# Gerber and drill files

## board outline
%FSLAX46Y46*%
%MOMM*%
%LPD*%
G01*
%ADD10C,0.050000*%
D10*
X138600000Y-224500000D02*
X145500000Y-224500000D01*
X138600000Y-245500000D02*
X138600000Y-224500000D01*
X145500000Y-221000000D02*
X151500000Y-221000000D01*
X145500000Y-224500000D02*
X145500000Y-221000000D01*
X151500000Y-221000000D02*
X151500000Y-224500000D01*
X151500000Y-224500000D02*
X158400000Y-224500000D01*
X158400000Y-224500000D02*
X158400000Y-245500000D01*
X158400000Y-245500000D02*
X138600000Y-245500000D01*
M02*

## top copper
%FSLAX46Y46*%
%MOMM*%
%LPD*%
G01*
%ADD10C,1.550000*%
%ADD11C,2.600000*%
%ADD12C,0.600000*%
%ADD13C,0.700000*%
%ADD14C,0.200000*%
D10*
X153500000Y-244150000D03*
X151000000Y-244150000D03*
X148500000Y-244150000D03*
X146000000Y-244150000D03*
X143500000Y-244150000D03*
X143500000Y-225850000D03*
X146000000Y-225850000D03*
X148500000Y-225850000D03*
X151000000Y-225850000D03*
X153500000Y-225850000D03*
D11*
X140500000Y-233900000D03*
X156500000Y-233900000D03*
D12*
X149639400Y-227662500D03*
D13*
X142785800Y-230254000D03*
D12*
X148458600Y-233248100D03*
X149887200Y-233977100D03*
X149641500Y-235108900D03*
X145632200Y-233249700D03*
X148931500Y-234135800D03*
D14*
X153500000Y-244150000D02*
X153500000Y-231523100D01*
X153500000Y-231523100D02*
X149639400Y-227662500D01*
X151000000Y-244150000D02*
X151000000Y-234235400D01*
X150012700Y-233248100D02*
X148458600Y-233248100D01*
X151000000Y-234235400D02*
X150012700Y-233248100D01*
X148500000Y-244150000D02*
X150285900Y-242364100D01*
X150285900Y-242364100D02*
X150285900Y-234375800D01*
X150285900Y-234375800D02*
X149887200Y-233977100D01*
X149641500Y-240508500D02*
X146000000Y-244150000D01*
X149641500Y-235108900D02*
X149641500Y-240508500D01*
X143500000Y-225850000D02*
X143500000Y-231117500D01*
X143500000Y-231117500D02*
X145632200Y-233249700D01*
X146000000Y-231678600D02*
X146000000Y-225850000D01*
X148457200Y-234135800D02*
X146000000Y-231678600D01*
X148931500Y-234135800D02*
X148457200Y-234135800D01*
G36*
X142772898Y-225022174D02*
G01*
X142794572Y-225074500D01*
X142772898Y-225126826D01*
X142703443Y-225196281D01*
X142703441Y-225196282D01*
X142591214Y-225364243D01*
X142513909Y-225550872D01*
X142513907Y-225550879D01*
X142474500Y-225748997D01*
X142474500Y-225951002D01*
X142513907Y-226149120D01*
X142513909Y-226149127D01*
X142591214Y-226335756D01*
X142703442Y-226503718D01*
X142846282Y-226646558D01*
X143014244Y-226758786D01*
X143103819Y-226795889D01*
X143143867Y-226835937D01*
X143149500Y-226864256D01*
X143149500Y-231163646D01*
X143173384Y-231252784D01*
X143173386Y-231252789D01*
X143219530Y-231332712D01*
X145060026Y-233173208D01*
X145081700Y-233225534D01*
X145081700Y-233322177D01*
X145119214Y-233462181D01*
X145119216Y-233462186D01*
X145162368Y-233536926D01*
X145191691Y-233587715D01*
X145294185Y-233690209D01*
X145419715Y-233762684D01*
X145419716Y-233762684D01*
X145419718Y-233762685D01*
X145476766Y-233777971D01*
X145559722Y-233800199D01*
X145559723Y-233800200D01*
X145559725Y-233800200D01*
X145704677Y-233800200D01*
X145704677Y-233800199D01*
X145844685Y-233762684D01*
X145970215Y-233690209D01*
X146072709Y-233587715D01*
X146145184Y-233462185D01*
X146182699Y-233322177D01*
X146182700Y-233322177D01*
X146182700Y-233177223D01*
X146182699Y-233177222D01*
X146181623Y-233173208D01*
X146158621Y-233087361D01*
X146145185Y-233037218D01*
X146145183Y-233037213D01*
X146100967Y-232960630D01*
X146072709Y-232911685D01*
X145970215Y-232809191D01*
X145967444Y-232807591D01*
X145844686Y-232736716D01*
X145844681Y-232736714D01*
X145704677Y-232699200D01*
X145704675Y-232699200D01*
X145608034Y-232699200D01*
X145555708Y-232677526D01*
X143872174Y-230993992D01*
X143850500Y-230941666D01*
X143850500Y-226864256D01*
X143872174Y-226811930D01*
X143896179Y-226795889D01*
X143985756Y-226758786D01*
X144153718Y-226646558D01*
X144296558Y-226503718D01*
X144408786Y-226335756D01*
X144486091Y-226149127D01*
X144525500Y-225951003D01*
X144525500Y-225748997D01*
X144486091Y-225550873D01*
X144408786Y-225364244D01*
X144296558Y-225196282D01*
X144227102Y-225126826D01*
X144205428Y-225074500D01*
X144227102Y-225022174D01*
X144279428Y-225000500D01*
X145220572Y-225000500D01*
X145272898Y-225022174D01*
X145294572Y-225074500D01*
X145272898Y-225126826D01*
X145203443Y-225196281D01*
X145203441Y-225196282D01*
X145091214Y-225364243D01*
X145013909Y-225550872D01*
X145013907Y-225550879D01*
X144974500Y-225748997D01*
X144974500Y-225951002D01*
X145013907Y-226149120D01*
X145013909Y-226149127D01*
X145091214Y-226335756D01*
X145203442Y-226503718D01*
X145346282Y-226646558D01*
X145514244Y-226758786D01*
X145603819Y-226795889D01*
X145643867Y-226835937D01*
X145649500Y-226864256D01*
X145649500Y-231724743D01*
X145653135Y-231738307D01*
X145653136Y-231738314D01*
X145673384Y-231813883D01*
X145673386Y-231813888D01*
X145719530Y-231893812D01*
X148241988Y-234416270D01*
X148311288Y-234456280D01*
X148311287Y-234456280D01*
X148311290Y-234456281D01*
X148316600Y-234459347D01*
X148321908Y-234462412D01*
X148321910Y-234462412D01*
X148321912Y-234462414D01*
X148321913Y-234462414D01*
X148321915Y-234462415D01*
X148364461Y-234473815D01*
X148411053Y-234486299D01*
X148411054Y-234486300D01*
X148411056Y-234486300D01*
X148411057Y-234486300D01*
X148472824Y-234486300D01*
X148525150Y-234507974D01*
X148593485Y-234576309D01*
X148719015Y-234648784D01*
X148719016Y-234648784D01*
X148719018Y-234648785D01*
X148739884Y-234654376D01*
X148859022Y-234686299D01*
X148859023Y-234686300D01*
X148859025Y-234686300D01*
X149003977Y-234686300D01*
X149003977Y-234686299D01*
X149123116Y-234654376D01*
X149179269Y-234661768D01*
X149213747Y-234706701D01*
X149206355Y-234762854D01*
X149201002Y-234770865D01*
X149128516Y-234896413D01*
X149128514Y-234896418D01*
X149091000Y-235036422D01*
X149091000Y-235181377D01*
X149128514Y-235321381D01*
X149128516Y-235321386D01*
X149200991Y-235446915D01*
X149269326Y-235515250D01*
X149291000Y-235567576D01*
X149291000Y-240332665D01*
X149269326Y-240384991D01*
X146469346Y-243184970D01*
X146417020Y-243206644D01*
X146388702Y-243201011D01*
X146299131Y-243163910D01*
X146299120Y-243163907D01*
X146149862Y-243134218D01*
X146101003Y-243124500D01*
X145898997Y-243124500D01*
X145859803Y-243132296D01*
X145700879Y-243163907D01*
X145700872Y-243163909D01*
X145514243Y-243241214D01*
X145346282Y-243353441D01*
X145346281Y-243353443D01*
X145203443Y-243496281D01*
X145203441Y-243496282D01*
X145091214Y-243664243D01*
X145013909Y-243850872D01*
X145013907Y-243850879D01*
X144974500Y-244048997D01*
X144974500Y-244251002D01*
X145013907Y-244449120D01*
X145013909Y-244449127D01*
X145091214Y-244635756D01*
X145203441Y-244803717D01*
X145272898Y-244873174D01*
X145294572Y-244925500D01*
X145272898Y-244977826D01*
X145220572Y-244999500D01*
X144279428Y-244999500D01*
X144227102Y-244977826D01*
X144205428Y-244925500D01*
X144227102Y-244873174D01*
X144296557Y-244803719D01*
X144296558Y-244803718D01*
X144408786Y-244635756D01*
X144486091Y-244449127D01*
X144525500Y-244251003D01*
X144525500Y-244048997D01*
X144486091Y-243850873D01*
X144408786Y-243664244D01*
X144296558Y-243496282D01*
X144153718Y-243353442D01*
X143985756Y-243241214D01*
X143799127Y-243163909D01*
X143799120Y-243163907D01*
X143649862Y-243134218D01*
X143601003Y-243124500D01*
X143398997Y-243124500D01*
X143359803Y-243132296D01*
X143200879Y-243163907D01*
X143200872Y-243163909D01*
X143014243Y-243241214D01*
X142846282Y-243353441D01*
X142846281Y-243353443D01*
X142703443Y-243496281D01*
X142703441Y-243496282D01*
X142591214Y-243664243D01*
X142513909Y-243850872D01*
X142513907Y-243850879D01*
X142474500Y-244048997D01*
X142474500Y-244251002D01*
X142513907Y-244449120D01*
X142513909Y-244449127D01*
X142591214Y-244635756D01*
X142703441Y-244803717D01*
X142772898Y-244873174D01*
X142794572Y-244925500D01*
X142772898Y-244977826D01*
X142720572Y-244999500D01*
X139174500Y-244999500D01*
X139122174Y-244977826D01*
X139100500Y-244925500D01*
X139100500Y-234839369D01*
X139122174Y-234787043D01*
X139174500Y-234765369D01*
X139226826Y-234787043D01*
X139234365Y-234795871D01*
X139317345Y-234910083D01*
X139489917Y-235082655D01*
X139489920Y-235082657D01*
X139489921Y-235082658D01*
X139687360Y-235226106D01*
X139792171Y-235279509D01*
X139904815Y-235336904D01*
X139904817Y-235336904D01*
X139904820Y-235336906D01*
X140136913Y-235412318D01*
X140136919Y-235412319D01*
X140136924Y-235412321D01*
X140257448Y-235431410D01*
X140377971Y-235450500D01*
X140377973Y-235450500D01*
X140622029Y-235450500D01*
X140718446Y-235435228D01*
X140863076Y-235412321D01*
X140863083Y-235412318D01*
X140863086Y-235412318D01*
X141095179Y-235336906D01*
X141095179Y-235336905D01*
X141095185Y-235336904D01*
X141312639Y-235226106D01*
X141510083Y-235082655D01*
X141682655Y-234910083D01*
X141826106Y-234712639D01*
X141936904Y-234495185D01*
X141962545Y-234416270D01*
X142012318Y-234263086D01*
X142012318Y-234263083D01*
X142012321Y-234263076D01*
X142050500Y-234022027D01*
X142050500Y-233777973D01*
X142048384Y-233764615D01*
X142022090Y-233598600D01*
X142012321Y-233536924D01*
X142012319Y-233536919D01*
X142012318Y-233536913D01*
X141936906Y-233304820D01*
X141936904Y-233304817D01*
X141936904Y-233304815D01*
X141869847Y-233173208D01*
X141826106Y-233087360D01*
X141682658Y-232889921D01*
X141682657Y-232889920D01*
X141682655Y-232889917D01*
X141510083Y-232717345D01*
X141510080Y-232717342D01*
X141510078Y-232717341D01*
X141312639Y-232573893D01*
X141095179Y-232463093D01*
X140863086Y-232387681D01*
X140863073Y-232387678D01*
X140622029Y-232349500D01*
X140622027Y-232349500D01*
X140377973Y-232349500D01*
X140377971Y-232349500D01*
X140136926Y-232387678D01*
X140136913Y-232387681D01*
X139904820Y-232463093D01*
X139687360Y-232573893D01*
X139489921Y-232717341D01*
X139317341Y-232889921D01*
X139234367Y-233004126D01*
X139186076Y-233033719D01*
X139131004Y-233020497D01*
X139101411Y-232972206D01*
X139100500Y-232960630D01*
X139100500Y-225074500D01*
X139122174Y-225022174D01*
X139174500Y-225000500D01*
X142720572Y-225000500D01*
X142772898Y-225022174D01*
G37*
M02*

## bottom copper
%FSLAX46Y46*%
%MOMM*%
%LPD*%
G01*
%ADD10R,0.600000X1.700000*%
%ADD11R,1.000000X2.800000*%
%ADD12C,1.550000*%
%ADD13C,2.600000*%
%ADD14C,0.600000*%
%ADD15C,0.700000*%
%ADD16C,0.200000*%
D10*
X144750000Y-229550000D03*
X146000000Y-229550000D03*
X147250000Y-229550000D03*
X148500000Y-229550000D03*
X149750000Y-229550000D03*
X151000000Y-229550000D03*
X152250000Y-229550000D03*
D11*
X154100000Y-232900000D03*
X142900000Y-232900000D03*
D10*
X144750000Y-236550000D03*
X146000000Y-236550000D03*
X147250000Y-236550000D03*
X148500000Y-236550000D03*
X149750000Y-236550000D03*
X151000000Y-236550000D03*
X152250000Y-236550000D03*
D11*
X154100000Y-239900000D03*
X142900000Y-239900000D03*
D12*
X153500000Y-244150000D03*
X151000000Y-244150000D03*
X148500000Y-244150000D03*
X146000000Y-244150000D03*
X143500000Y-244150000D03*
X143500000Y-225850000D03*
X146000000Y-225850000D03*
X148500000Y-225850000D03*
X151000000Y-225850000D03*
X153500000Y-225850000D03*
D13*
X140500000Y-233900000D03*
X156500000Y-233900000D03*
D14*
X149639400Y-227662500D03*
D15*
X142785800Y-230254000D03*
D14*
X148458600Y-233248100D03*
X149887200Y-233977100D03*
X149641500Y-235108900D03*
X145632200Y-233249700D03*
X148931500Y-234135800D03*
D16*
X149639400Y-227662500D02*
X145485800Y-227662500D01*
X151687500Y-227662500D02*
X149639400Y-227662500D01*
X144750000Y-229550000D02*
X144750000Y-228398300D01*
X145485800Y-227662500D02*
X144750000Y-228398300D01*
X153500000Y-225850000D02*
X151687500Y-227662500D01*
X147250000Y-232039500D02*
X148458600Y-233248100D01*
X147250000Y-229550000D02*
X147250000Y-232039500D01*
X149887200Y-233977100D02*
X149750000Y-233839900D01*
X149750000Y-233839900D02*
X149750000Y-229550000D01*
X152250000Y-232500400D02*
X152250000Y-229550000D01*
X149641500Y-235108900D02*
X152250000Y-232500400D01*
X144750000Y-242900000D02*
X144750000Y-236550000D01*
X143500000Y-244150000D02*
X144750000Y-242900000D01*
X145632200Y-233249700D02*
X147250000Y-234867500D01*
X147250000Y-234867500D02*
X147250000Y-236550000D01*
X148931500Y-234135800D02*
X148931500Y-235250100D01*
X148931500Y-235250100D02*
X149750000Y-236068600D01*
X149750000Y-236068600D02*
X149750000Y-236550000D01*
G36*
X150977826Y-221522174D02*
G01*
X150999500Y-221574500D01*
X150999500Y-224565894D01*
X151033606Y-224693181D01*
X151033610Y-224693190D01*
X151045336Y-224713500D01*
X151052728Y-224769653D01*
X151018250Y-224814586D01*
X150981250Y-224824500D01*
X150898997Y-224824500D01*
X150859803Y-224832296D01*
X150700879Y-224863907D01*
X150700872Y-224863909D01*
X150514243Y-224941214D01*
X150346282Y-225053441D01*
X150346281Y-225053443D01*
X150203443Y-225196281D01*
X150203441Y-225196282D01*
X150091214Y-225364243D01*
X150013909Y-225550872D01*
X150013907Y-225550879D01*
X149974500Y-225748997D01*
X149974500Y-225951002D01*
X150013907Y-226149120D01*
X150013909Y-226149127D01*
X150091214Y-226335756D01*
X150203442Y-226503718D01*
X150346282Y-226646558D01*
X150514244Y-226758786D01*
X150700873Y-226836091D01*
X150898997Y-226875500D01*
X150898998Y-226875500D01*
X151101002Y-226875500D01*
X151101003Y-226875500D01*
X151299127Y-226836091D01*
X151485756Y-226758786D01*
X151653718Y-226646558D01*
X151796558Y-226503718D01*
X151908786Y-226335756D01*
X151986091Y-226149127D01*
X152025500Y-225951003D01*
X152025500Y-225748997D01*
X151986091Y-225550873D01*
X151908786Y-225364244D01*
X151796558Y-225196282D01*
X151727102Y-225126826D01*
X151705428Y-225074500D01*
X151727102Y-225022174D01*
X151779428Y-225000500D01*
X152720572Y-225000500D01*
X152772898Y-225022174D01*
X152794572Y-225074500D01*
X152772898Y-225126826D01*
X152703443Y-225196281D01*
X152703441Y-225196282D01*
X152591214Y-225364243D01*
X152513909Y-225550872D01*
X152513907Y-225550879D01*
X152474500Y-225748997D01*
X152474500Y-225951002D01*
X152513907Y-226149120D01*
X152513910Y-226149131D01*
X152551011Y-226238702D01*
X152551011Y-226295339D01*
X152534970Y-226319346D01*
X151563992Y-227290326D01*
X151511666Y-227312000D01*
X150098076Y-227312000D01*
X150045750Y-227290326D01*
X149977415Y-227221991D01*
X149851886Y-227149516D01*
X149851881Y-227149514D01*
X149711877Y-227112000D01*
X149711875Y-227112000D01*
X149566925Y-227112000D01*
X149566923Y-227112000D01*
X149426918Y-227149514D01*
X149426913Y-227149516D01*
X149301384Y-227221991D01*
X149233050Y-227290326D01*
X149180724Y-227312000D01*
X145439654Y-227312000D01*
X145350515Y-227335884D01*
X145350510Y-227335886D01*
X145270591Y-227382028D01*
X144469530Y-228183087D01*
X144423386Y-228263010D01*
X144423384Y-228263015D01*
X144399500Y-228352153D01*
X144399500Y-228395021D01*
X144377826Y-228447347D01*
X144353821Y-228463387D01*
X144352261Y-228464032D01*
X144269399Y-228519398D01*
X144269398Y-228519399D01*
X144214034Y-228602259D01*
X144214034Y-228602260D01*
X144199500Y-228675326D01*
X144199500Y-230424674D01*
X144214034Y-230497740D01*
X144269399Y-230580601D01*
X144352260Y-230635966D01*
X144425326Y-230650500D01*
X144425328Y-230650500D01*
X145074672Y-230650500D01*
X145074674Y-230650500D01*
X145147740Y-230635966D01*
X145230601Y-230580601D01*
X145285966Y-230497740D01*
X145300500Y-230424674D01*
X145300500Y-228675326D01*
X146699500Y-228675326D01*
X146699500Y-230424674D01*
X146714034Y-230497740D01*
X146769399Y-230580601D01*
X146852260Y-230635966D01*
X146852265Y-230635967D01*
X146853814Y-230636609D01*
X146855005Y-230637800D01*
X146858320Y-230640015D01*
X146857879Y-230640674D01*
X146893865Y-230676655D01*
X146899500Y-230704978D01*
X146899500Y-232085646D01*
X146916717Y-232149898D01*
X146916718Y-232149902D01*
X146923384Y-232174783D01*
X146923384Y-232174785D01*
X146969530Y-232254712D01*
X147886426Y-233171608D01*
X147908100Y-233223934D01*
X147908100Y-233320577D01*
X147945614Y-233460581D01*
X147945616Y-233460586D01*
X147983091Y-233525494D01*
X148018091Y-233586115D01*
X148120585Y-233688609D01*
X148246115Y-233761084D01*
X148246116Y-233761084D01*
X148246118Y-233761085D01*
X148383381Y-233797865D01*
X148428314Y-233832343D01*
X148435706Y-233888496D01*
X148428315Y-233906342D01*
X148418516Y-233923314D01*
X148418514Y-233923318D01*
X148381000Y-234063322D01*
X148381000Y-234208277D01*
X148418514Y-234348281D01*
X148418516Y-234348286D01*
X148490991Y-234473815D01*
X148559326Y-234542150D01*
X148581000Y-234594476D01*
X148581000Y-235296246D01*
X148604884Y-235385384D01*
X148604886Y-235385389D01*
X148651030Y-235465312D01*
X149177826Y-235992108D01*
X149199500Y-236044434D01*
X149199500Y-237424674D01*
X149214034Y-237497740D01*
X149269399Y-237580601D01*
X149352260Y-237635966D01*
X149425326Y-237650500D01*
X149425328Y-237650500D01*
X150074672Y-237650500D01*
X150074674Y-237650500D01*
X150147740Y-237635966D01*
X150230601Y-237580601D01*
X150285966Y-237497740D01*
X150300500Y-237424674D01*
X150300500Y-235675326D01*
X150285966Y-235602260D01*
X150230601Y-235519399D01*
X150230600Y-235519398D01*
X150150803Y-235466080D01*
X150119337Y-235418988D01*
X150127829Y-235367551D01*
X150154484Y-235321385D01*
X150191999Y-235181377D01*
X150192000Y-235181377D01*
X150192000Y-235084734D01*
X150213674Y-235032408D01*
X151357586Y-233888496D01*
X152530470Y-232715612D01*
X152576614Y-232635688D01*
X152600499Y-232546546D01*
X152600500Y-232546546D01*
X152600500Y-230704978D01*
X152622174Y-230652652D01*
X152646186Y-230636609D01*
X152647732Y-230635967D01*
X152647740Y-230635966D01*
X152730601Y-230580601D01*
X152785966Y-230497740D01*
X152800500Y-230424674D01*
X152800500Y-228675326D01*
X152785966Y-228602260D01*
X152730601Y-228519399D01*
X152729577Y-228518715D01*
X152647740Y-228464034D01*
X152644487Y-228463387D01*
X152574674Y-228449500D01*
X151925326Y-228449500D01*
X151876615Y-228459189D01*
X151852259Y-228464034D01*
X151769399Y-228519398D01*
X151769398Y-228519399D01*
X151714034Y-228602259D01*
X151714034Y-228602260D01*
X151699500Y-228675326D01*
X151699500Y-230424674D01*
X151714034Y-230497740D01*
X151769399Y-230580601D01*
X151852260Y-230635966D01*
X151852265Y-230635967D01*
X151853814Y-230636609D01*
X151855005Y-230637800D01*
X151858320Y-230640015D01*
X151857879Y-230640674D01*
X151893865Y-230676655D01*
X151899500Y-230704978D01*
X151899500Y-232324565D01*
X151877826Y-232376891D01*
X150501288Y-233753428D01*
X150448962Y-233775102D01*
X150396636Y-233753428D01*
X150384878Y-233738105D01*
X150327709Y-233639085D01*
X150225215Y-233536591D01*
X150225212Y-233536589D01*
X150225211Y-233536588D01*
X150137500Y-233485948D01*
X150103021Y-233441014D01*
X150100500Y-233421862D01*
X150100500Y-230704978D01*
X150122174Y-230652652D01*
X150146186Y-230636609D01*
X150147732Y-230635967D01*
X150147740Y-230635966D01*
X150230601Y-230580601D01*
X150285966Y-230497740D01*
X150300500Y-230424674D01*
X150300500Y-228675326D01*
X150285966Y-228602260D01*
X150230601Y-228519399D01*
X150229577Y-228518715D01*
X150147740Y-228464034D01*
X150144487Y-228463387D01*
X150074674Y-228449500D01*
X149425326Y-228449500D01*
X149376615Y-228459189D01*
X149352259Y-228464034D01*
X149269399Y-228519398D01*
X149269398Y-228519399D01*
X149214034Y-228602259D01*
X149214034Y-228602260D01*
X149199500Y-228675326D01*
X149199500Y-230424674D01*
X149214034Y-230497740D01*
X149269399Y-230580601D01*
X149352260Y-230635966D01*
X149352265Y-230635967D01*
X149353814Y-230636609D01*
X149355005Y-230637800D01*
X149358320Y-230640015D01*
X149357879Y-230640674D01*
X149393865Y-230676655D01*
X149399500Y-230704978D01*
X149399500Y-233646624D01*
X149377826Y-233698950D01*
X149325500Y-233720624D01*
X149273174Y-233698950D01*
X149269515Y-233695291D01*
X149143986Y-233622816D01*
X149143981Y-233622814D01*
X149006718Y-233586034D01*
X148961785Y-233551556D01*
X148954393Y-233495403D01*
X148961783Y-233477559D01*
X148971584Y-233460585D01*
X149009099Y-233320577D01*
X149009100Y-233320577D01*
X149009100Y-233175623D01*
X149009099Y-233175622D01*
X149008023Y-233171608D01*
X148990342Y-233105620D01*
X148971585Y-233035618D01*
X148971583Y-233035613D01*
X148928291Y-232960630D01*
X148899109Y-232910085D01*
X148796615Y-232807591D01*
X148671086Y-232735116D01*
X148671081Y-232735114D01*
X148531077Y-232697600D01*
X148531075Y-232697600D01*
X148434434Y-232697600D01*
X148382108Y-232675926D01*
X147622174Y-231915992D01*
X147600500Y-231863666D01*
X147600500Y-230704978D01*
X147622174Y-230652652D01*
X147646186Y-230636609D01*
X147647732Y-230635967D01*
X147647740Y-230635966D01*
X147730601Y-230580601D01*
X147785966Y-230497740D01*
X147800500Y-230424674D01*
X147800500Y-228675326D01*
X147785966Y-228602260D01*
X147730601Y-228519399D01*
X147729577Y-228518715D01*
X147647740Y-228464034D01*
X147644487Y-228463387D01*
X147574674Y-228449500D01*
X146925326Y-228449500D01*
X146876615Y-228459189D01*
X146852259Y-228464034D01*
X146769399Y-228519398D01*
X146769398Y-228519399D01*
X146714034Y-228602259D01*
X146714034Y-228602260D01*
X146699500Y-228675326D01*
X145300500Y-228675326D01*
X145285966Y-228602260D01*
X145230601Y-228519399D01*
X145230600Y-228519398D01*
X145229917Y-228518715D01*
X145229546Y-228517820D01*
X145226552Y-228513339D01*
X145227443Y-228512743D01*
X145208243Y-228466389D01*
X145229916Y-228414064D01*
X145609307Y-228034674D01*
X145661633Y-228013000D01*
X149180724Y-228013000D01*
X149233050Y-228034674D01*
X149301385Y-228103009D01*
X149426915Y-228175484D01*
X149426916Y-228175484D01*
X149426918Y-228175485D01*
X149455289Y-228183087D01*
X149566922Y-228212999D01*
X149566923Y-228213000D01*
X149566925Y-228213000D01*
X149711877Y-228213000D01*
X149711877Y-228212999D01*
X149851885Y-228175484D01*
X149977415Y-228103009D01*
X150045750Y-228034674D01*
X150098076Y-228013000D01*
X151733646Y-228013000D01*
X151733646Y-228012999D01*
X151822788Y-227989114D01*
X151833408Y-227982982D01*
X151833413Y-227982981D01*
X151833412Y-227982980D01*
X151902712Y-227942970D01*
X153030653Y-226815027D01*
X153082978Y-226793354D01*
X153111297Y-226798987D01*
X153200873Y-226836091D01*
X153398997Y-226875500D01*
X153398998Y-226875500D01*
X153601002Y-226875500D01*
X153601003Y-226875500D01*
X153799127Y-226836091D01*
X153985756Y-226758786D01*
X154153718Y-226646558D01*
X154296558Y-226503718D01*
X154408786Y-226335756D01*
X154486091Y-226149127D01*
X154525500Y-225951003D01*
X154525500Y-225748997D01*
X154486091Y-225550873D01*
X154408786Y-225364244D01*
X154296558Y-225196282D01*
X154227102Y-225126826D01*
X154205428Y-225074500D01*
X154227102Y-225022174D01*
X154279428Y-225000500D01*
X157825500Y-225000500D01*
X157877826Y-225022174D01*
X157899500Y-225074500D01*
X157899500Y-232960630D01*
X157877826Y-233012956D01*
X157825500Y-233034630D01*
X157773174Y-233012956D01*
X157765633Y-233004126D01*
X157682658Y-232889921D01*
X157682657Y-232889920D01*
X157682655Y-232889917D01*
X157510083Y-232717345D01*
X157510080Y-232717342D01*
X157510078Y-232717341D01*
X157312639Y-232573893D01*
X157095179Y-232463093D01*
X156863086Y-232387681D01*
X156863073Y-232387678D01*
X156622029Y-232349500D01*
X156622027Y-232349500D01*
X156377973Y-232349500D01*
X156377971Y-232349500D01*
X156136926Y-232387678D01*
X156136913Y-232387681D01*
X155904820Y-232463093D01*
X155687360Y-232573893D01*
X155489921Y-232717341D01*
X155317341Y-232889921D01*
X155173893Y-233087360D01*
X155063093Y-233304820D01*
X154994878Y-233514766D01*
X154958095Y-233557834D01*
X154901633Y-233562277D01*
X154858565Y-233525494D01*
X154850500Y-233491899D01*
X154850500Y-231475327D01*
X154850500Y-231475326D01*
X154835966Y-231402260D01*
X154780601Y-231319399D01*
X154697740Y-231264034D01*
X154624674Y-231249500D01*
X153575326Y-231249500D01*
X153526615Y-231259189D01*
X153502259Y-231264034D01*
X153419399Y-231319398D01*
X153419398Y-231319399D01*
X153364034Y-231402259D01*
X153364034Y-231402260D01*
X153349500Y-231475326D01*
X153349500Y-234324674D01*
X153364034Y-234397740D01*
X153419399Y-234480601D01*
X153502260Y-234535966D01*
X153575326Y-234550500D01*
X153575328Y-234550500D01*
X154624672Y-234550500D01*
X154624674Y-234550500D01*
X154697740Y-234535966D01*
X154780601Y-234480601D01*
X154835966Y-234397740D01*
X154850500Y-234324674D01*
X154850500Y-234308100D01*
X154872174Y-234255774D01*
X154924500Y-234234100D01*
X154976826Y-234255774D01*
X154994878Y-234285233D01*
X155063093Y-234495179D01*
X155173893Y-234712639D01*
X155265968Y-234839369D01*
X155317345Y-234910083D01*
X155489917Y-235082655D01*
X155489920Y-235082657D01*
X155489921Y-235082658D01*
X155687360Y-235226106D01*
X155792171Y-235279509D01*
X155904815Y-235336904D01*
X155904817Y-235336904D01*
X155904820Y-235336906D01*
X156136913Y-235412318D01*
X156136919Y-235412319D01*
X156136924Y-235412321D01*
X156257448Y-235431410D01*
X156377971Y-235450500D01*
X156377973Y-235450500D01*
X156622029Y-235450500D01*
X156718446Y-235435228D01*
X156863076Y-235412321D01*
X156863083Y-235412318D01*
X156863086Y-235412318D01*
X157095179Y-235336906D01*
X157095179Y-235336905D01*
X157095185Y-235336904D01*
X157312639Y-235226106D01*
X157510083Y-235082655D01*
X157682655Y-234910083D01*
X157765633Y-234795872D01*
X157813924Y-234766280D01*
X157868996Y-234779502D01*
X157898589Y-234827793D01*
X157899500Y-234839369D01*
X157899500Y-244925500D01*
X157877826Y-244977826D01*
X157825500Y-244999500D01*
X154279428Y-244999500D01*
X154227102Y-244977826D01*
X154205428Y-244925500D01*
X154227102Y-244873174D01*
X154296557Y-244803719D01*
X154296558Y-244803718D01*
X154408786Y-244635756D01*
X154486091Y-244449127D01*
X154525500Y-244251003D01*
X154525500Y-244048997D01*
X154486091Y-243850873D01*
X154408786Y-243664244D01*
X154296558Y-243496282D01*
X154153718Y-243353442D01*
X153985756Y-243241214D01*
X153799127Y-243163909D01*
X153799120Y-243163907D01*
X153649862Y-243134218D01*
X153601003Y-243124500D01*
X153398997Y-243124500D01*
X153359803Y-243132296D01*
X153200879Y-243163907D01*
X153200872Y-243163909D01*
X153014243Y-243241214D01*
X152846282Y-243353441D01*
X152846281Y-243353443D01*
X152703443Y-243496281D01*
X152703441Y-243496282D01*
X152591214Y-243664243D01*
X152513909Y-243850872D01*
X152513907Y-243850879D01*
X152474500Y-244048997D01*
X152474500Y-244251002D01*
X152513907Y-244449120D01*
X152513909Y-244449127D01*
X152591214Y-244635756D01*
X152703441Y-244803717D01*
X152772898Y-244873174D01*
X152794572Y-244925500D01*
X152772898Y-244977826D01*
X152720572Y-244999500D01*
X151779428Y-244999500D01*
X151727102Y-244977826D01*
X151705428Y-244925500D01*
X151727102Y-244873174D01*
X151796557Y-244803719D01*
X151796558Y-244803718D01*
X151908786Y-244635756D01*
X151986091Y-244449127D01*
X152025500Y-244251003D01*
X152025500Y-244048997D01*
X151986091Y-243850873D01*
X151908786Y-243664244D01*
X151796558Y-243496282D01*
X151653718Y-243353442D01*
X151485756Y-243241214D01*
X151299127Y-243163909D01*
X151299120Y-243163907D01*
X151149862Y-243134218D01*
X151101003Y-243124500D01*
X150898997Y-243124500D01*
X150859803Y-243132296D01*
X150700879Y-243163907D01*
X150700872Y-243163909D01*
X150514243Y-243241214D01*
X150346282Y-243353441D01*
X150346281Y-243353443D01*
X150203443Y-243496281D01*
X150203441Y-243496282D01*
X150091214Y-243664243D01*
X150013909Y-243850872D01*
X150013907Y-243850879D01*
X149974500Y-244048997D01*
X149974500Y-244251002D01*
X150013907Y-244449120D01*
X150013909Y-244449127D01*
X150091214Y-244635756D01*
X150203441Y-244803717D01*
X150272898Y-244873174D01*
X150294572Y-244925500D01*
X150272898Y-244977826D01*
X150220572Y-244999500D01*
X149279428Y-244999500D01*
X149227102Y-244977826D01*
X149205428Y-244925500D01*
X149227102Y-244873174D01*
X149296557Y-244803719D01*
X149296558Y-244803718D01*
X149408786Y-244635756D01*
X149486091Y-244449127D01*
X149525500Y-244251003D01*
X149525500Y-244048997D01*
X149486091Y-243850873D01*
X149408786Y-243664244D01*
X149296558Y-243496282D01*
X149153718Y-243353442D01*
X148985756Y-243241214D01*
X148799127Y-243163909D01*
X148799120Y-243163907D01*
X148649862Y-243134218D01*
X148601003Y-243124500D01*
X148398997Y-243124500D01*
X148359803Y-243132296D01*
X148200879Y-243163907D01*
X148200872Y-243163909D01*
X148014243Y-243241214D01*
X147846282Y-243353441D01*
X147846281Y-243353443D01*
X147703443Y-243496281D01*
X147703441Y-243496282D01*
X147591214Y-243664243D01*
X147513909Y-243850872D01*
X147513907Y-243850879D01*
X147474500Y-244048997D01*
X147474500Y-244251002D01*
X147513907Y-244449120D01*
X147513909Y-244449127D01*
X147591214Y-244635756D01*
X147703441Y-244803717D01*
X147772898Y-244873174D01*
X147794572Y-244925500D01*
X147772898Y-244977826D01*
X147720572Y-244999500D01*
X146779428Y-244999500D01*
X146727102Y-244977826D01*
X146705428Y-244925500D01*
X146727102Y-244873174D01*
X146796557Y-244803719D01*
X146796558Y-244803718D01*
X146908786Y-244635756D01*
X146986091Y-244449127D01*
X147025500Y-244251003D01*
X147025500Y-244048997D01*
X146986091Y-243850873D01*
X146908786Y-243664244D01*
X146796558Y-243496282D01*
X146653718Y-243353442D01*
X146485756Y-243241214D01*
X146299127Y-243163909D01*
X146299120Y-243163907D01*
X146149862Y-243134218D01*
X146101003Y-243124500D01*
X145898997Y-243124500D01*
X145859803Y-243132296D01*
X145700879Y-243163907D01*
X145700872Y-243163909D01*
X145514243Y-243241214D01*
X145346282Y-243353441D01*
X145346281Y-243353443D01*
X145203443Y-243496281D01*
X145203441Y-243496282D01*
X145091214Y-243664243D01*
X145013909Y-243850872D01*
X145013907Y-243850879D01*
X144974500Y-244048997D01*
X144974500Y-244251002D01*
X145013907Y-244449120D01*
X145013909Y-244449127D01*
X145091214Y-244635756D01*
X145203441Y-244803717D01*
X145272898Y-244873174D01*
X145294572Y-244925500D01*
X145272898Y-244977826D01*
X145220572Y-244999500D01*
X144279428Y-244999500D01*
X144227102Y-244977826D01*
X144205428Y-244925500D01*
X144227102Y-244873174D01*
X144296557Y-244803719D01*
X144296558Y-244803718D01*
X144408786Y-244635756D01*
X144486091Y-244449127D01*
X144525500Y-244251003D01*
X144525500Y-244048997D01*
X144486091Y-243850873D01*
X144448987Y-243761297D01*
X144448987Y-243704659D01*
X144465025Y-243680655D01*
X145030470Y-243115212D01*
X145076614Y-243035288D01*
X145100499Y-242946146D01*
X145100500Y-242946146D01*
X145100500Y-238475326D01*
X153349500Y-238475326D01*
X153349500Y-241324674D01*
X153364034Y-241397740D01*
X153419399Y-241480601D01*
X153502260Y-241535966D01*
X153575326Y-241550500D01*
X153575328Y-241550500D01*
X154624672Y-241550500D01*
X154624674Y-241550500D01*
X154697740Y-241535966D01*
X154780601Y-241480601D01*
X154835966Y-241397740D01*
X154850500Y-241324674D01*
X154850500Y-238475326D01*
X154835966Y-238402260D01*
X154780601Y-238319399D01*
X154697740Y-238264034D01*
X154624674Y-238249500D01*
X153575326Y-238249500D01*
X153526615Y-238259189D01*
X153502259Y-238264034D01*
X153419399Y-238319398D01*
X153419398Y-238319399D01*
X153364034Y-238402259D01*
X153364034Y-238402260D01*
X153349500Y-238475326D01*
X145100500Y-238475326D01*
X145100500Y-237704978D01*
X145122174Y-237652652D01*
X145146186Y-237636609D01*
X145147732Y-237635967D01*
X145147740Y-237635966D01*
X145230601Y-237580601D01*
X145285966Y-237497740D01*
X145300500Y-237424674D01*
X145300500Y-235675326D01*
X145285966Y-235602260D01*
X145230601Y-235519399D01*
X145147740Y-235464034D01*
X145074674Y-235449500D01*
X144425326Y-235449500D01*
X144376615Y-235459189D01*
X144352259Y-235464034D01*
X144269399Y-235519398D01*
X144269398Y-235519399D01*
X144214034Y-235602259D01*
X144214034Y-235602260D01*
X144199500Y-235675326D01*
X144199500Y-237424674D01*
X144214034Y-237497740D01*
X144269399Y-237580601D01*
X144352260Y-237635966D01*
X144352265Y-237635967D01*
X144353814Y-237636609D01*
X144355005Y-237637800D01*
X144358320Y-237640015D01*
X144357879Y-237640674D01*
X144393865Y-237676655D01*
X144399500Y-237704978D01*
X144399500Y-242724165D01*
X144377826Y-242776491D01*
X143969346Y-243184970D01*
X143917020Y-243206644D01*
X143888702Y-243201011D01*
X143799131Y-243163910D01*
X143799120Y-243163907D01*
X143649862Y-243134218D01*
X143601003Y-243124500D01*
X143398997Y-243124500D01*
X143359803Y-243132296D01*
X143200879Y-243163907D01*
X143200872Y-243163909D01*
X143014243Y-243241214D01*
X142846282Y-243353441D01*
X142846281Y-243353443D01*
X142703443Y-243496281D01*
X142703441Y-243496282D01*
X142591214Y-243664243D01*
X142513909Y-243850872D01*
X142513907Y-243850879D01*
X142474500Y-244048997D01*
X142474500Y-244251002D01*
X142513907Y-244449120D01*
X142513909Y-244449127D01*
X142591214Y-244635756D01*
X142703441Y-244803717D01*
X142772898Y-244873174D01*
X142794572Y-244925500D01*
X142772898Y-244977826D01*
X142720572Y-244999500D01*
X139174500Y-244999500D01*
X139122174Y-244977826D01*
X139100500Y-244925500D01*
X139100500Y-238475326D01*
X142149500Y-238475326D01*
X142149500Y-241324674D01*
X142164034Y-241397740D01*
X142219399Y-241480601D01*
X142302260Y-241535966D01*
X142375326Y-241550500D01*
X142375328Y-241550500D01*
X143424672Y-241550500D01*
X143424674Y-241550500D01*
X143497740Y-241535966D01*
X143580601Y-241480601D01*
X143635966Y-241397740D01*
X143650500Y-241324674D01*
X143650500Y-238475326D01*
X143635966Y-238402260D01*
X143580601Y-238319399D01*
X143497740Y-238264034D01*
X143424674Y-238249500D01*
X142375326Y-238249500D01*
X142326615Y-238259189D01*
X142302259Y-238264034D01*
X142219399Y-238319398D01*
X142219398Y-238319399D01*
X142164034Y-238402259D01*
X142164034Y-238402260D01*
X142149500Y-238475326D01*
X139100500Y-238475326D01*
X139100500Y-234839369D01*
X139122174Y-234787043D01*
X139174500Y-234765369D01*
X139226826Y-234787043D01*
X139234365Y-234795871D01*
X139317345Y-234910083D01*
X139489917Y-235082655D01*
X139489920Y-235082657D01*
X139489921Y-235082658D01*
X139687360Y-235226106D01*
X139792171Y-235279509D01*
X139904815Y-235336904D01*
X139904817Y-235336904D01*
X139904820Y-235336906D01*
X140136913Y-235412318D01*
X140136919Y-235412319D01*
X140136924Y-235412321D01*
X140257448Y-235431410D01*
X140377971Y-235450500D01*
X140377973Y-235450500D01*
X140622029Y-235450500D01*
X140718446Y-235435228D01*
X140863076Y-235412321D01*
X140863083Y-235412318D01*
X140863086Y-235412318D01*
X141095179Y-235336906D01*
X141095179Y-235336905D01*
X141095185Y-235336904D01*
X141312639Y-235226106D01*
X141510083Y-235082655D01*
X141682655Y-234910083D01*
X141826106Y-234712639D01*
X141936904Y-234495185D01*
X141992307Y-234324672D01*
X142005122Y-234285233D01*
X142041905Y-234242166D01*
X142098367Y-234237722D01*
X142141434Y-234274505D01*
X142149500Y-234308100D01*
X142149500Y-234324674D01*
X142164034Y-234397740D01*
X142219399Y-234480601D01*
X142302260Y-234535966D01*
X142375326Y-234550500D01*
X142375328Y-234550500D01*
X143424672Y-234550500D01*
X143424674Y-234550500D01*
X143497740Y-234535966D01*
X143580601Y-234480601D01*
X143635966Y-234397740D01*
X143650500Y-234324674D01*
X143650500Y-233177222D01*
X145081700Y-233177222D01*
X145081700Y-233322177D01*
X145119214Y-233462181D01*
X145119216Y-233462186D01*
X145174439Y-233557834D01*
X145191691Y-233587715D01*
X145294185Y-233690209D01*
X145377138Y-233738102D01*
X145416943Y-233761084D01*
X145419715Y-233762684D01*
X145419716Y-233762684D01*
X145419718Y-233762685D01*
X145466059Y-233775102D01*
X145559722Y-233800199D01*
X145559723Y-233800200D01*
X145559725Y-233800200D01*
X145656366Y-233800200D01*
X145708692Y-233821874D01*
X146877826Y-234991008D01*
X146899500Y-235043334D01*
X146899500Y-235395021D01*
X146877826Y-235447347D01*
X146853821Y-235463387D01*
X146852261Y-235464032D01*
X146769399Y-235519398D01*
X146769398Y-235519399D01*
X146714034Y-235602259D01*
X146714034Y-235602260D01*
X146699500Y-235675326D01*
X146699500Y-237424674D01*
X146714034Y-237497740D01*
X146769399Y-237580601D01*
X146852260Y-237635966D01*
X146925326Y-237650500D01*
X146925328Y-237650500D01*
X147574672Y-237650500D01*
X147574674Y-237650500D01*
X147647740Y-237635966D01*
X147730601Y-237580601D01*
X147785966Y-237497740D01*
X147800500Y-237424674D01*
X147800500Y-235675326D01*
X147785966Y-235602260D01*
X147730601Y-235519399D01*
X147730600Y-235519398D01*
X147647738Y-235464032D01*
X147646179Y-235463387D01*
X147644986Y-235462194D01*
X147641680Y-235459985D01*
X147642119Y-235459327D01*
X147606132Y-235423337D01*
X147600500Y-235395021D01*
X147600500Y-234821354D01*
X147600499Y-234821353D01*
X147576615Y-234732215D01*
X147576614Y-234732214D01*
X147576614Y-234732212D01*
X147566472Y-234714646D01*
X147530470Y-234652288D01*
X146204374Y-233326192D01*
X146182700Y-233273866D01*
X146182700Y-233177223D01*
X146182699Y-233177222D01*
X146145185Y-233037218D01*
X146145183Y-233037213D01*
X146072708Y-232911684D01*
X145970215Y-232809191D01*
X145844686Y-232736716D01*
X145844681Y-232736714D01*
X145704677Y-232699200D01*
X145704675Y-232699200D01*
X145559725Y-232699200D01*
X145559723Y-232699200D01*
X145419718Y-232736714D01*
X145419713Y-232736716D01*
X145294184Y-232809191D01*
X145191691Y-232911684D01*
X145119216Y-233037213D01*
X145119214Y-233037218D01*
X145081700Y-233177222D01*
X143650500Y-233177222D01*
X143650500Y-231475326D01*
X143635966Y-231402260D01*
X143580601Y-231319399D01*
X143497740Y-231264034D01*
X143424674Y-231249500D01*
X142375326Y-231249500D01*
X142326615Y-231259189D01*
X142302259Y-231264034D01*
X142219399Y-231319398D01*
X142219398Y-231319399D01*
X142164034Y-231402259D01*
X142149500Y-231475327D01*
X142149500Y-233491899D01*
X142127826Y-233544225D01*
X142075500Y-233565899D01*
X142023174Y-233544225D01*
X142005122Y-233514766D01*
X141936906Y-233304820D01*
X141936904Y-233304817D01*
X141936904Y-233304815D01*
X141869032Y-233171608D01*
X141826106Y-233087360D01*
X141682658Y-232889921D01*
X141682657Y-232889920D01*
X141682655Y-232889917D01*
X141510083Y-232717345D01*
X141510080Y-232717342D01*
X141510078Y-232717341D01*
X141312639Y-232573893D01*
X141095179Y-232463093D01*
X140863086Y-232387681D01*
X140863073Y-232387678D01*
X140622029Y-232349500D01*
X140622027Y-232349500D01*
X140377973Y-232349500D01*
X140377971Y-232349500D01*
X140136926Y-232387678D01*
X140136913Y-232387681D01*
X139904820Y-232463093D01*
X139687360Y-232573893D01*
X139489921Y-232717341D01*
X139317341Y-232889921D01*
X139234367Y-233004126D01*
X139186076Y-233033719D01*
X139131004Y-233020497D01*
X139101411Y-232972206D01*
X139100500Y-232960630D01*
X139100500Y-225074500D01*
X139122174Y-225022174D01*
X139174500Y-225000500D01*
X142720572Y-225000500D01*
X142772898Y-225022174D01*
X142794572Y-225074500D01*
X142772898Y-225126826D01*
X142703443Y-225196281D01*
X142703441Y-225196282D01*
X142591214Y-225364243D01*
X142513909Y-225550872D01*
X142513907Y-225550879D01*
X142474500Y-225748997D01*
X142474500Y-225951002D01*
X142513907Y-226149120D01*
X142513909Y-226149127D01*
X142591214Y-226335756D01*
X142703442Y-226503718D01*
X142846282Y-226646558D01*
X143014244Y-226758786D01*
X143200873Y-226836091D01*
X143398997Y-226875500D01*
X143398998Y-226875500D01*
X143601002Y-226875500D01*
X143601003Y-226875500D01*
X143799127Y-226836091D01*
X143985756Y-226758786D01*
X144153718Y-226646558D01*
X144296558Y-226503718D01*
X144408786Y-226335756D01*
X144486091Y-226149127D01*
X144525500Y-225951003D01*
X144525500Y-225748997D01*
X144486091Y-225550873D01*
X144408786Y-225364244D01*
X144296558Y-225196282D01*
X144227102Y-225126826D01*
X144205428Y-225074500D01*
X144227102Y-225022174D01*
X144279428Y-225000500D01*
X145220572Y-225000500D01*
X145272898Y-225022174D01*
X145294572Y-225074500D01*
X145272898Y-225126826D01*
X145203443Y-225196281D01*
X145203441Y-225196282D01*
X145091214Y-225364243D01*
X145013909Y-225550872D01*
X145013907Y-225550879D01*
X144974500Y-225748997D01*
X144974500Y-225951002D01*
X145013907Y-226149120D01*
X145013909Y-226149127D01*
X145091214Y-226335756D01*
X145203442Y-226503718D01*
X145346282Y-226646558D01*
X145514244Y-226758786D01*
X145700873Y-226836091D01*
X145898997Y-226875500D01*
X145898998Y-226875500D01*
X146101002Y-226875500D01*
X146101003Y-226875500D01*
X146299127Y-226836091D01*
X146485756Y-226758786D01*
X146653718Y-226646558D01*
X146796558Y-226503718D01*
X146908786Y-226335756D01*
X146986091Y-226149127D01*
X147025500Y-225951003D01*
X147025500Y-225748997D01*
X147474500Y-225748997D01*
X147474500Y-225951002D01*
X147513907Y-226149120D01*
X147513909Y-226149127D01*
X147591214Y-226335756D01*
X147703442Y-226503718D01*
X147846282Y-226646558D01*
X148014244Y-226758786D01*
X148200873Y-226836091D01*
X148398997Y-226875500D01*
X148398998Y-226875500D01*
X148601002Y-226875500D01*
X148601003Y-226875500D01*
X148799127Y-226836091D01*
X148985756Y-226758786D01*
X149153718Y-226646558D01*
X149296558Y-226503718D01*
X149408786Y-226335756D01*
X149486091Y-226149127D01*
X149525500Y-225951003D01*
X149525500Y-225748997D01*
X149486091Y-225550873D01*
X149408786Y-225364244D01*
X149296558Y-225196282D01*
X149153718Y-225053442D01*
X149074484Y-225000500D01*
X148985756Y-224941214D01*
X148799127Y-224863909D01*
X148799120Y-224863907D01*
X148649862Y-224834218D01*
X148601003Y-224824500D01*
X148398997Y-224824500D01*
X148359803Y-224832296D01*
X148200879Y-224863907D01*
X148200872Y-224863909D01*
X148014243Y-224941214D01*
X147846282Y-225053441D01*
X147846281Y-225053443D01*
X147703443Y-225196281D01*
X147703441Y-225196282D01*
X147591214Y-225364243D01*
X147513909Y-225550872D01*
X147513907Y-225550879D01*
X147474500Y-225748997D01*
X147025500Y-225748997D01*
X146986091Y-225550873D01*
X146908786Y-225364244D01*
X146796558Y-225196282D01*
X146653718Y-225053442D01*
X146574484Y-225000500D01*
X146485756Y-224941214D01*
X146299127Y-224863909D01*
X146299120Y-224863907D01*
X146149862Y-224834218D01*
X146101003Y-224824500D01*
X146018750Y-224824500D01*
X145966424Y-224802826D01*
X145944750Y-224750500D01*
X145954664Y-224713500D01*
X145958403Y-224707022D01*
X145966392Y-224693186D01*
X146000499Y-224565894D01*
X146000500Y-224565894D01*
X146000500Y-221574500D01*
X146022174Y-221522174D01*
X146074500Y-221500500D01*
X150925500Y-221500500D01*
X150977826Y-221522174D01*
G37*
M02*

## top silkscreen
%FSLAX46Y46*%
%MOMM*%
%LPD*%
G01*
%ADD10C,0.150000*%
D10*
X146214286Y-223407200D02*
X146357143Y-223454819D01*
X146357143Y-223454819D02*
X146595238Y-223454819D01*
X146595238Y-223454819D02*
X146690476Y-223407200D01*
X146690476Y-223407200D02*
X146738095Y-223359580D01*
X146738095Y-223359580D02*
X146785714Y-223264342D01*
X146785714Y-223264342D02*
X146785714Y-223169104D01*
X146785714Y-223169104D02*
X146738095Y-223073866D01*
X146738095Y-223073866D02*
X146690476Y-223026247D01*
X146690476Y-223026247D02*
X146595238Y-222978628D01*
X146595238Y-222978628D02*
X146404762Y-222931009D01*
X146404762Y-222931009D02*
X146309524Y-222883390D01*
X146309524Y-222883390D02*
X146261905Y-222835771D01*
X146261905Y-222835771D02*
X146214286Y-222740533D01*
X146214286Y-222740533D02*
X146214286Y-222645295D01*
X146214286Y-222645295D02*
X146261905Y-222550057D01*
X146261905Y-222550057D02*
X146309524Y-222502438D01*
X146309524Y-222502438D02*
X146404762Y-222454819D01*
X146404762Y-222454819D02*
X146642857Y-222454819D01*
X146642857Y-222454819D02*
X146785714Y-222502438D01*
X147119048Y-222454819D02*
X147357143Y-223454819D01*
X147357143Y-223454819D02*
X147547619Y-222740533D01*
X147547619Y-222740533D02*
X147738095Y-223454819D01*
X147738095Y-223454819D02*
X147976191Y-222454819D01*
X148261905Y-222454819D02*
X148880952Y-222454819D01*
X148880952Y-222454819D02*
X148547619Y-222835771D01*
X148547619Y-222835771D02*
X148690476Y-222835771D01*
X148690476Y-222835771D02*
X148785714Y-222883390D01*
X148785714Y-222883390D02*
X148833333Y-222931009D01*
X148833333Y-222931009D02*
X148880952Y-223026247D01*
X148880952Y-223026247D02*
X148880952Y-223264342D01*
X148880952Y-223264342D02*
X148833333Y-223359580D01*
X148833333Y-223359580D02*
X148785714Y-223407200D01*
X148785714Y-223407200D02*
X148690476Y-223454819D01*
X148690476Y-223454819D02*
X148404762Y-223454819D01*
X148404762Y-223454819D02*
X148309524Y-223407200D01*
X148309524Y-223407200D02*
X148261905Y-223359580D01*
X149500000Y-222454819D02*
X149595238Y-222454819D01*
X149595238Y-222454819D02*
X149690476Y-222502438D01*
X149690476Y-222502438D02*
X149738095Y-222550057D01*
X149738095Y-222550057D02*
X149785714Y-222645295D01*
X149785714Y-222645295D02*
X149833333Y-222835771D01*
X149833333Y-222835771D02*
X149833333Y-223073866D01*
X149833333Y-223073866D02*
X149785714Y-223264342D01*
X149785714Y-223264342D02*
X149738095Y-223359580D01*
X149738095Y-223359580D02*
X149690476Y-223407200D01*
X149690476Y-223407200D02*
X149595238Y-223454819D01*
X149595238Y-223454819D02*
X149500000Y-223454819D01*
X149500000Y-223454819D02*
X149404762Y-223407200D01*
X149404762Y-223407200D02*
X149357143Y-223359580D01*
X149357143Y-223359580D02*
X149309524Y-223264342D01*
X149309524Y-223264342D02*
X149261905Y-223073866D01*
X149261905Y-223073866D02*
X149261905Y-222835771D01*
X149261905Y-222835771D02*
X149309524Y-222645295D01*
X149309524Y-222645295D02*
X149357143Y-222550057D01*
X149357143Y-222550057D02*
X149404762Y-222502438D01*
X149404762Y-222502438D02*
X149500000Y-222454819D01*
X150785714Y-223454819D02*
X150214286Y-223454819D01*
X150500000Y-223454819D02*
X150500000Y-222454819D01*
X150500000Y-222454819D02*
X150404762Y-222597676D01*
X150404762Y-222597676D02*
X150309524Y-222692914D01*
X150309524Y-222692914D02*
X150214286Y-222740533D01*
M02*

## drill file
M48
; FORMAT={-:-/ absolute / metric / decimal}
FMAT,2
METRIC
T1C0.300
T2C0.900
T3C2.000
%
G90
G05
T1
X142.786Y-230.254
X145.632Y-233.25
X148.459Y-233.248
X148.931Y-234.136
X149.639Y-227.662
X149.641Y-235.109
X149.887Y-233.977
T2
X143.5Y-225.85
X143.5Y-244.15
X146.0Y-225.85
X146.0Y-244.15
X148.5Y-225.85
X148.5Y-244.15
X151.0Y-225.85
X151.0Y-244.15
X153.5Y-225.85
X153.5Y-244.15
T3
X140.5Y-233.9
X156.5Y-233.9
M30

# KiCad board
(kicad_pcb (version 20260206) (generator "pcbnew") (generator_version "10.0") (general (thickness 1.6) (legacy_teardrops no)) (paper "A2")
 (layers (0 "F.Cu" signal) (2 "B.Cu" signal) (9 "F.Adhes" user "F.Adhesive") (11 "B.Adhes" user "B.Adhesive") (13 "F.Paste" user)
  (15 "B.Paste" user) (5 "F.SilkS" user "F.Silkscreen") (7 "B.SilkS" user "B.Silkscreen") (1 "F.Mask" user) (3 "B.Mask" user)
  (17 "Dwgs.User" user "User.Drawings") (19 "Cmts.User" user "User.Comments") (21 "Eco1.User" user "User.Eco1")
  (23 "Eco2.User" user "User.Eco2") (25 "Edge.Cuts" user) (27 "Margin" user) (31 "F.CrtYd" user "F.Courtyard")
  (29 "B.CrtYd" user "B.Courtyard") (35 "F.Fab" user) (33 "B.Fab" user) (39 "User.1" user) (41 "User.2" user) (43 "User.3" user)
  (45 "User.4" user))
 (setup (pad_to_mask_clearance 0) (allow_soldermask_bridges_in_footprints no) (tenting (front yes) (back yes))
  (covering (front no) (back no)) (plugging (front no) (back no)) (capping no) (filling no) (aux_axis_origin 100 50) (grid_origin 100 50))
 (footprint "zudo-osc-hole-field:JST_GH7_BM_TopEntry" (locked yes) (layer "B.Cu") (at 148.5 229.55 180)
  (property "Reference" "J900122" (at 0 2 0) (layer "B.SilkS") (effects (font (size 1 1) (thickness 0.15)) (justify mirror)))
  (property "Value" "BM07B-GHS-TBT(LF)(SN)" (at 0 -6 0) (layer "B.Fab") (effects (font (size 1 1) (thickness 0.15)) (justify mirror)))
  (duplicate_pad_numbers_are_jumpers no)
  (pad "1" smd rect (at 3.75 0 180) (size 0.6 1.7) (layers "B.Cu" "B.Mask" "B.Paste") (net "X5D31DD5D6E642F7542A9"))
  (pad "2" smd rect (at 2.5 0 180) (size 0.6 1.7) (layers "B.Cu" "B.Mask" "B.Paste") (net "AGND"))
  (pad "3" smd rect (at 1.25 0 180) (size 0.6 1.7) (layers "B.Cu" "B.Mask" "B.Paste") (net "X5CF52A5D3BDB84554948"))
  (pad "4" smd rect (at 0 0 180) (size 0.6 1.7) (layers "B.Cu" "B.Mask" "B.Paste") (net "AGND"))
  (pad "5" smd rect (at -1.25 0 180) (size 0.6 1.7) (layers "B.Cu" "B.Mask" "B.Paste") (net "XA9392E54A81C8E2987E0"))
  (pad "6" smd rect (at -2.5 0 180) (size 0.6 1.7) (layers "B.Cu" "B.Mask" "B.Paste") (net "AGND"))
  (pad "7" smd rect (at -3.75 0 180) (size 0.6 1.7) (layers "B.Cu" "B.Mask" "B.Paste") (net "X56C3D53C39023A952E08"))
  (pad "MP1" smd rect (at -5.6 -3.35 180) (size 1 2.8) (layers "B.Cu" "B.Mask" "B.Paste") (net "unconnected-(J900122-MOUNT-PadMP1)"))
  (pad "MP2" smd rect (at 5.6 -3.35 180) (size 1 2.8) (layers "B.Cu" "B.Mask" "B.Paste") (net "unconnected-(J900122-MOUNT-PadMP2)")))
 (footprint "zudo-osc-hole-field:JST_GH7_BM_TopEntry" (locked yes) (layer "B.Cu") (at 148.5 236.55 180)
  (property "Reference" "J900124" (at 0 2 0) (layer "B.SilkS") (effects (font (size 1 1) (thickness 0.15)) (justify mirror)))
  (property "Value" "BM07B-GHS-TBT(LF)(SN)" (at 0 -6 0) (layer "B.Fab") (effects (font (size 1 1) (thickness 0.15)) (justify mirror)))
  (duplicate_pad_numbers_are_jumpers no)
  (pad "1" smd rect (at 3.75 0 180) (size 0.6 1.7) (layers "B.Cu" "B.Mask" "B.Paste") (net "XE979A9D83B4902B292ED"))
  (pad "2" smd rect (at 2.5 0 180) (size 0.6 1.7) (layers "B.Cu" "B.Mask" "B.Paste") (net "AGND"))
  (pad "3" smd rect (at 1.25 0 180) (size 0.6 1.7) (layers "B.Cu" "B.Mask" "B.Paste") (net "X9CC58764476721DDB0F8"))
  (pad "4" smd rect (at 0 0 180) (size 0.6 1.7) (layers "B.Cu" "B.Mask" "B.Paste") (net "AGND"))
  (pad "5" smd rect (at -1.25 0 180) (size 0.6 1.7) (layers "B.Cu" "B.Mask" "B.Paste") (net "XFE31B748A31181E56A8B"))
  (pad "6" smd rect (at -2.5 0 180) (size 0.6 1.7) (layers "B.Cu" "B.Mask" "B.Paste") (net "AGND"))
  (pad "7" smd rect (at -3.75 0 180) (size 0.6 1.7) (layers "B.Cu" "B.Mask" "B.Paste") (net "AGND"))
  (pad "MP1" smd rect (at -5.6 -3.35 180) (size 1 2.8) (layers "B.Cu" "B.Mask" "B.Paste") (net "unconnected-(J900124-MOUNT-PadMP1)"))
  (pad "MP2" smd rect (at 5.6 -3.35 180) (size 1 2.8) (layers "B.Cu" "B.Mask" "B.Paste") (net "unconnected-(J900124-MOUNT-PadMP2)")))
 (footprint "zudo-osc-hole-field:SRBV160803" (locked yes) (layer "F.Cu") (at 148.5 235)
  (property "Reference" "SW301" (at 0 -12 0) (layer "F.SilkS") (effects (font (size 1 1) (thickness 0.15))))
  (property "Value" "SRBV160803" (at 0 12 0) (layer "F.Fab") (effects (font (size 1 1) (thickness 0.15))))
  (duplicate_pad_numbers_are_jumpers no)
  (pad "1" thru_hole circle (at 5 9.15) (size 1.55 1.55) (drill 0.9) (layers "*.Cu" "*.Mask") (remove_unused_layers no)
   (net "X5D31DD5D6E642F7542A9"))
  (pad "2" thru_hole circle (at 2.5 9.15) (size 1.55 1.55) (drill 0.9) (layers "*.Cu" "*.Mask") (remove_unused_layers no)
   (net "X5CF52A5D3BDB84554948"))
  (pad "3" thru_hole circle (at 0 9.15) (size 1.55 1.55) (drill 0.9) (layers "*.Cu" "*.Mask") (remove_unused_layers no)
   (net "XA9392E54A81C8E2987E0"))
  (pad "4" thru_hole circle (at -2.5 9.15) (size 1.55 1.55) (drill 0.9) (layers "*.Cu" "*.Mask") (remove_unused_layers no)
   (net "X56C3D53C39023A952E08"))
  (pad "5" thru_hole circle (at -5 9.15) (size 1.55 1.55) (drill 0.9) (layers "*.Cu" "*.Mask") (remove_unused_layers no)
   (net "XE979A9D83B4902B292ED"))
  (pad "6" thru_hole circle (at -5 -9.15) (size 1.55 1.55) (drill 0.9) (layers "*.Cu" "*.Mask") (remove_unused_layers no)
   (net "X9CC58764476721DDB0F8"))
  (pad "7" thru_hole circle (at -2.5 -9.15) (size 1.55 1.55) (drill 0.9) (layers "*.Cu" "*.Mask") (remove_unused_layers no)
   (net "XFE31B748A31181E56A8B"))
  (pad "8" thru_hole circle (at 0 -9.15) (size 1.55 1.55) (drill 0.9) (layers "*.Cu" "*.Mask") (remove_unused_layers no)
   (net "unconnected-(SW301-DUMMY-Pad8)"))
  (pad "9" thru_hole circle (at 2.5 -9.15) (size 1.55 1.55) (drill 0.9) (layers "*.Cu" "*.Mask") (remove_unused_layers no)
   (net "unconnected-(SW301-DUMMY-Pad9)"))
  (pad "10" thru_hole circle (at 5 -9.15) (size 1.55 1.55) (drill 0.9) (layers "*.Cu" "*.Mask") (remove_unused_layers no)
   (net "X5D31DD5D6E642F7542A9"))
  (pad "MP1" thru_hole circle (at -8 -1.1) (size 2.6 2.6) (drill 2) (layers "*.Cu" "*.Mask") (remove_unused_layers no)
   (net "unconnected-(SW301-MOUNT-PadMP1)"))
  (pad "MP2" thru_hole circle (at 8 -1.1) (size 2.6 2.6) (drill 2) (layers "*.Cu" "*.Mask") (remove_unused_layers no)
   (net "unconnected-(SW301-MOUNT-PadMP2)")))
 (gr_line (start 138.6 224.5) (end 145.5 224.5) (stroke (width 0.05) (type default)) (layer "Edge.Cuts"))
 (gr_line (start 138.6 245.5) (end 138.6 224.5) (stroke (width 0.05) (type default)) (layer "Edge.Cuts"))
 (gr_line (start 145.5 221) (end 151.5 221) (stroke (width 0.05) (type default)) (layer "Edge.Cuts"))
 (gr_line (start 145.5 224.5) (end 145.5 221) (stroke (width 0.05) (type default)) (layer "Edge.Cuts"))
 (gr_line (start 151.5 221) (end 151.5 224.5) (stroke (width 0.05) (type default)) (layer "Edge.Cuts"))
 (gr_line (start 151.5 224.5) (end 158.4 224.5) (stroke (width 0.05) (type default)) (layer "Edge.Cuts"))
 (gr_line (start 158.4 224.5) (end 158.4 245.5) (stroke (width 0.05) (type default)) (layer "Edge.Cuts"))
 (gr_line (start 158.4 245.5) (end 138.6 245.5) (stroke (width 0.05) (type default)) (layer "Edge.Cuts"))
 (segment (start 153.5 244.15) (end 153.5 231.5231) (width 0.2) (layer "F.Cu") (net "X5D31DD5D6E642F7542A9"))
 (segment (start 153.5 231.5231) (end 149.6394 227.6625) (width 0.2) (layer "F.Cu") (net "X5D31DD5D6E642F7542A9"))
 (via (at 149.6394 227.6625) (size 0.6) (drill 0.3) (layers "F.Cu" "B.Cu") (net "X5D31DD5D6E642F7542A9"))
 (segment (start 149.6394 227.6625) (end 145.4858 227.6625) (width 0.2) (layer "B.Cu") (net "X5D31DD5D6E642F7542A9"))
 (segment (start 151.6875 227.6625) (end 149.6394 227.6625) (width 0.2) (layer "B.Cu") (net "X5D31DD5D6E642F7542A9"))
 (segment (start 144.75 229.55) (end 144.75 228.3983) (width 0.2) (layer "B.Cu") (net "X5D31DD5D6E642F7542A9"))
 (segment (start 145.4858 227.6625) (end 144.75 228.3983) (width 0.2) (layer "B.Cu") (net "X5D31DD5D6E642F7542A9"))
 (segment (start 153.5 225.85) (end 151.6875 227.6625) (width 0.2) (layer "B.Cu") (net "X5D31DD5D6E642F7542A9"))
 (via (at 142.7858 230.254) (size 0.7) (drill 0.3) (layers "F.Cu" "B.Cu") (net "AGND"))
 (segment (start 151 244.15) (end 151 234.2354) (width 0.2) (layer "F.Cu") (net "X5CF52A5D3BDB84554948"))
 (segment (start 150.0127 233.2481) (end 148.4586 233.2481) (width 0.2) (layer "F.Cu") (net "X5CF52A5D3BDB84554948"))
 (segment (start 151 234.2354) (end 150.0127 233.2481) (width 0.2) (layer "F.Cu") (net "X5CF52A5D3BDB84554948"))
 (via (at 148.4586 233.2481) (size 0.6) (drill 0.3) (layers "F.Cu" "B.Cu") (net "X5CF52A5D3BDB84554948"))
 (segment (start 147.25 232.0395) (end 148.4586 233.2481) (width 0.2) (layer "B.Cu") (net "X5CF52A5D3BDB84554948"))
 (segment (start 147.25 229.55) (end 147.25 232.0395) (width 0.2) (layer "B.Cu") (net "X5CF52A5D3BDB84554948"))
 (segment (start 148.5 244.15) (end 150.2859 242.3641) (width 0.2) (layer "F.Cu") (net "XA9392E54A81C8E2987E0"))
 (segment (start 150.2859 242.3641) (end 150.2859 234.3758) (width 0.2) (layer "F.Cu") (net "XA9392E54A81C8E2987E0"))
 (segment (start 150.2859 234.3758) (end 149.8872 233.9771) (width 0.2) (layer "F.Cu") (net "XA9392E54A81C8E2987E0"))
 (via (at 149.8872 233.9771) (size 0.6) (drill 0.3) (layers "F.Cu" "B.Cu") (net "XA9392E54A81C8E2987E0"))
 (segment (start 149.8872 233.9771) (end 149.75 233.8399) (width 0.2) (layer "B.Cu") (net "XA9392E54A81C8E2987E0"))
 (segment (start 149.75 233.8399) (end 149.75 229.55) (width 0.2) (layer "B.Cu") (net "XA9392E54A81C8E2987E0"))
 (segment (start 149.6415 240.5085) (end 146 244.15) (width 0.2) (layer "F.Cu") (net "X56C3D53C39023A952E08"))
 (segment (start 149.6415 235.1089) (end 149.6415 240.5085) (width 0.2) (layer "F.Cu") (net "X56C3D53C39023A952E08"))
 (via (at 149.6415 235.1089) (size 0.6) (drill 0.3) (layers "F.Cu" "B.Cu") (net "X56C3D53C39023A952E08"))
 (segment (start 152.25 232.5004) (end 152.25 229.55) (width 0.2) (layer "B.Cu") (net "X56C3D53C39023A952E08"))
 (segment (start 149.6415 235.1089) (end 152.25 232.5004) (width 0.2) (layer "B.Cu") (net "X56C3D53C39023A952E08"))
 (segment (start 144.75 242.9) (end 144.75 236.55) (width 0.2) (layer "B.Cu") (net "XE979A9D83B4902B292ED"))
 (segment (start 143.5 244.15) (end 144.75 242.9) (width 0.2) (layer "B.Cu") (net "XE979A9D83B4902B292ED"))
 (segment (start 143.5 225.85) (end 143.5 231.1175) (width 0.2) (layer "F.Cu") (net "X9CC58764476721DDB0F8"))
 (segment (start 143.5 231.1175) (end 145.6322 233.2497) (width 0.2) (layer "F.Cu") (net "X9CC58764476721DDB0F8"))
 (via (at 145.6322 233.2497) (size 0.6) (drill 0.3) (layers "F.Cu" "B.Cu") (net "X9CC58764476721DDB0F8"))
 (segment (start 145.6322 233.2497) (end 147.25 234.8675) (width 0.2) (layer "B.Cu") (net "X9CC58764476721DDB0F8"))
 (segment (start 147.25 234.8675) (end 147.25 236.55) (width 0.2) (layer "B.Cu") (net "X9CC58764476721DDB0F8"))
 (segment (start 146 231.6786) (end 146 225.85) (width 0.2) (layer "F.Cu") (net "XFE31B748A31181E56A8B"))
 (segment (start 148.4572 234.1358) (end 146 231.6786) (width 0.2) (layer "F.Cu") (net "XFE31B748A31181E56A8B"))
 (segment (start 148.9315 234.1358) (end 148.4572 234.1358) (width 0.2) (layer "F.Cu") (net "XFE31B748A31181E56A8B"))
 (via (at 148.9315 234.1358) (size 0.6) (drill 0.3) (layers "F.Cu" "B.Cu") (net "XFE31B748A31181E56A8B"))
 (segment (start 148.9315 234.1358) (end 148.9315 235.2501) (width 0.2) (layer "B.Cu") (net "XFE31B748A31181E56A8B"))
 (segment (start 148.9315 235.2501) (end 149.75 236.0686) (width 0.2) (layer "B.Cu") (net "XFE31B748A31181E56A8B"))
 (segment (start 149.75 236.0686) (end 149.75 236.55) (width 0.2) (layer "B.Cu") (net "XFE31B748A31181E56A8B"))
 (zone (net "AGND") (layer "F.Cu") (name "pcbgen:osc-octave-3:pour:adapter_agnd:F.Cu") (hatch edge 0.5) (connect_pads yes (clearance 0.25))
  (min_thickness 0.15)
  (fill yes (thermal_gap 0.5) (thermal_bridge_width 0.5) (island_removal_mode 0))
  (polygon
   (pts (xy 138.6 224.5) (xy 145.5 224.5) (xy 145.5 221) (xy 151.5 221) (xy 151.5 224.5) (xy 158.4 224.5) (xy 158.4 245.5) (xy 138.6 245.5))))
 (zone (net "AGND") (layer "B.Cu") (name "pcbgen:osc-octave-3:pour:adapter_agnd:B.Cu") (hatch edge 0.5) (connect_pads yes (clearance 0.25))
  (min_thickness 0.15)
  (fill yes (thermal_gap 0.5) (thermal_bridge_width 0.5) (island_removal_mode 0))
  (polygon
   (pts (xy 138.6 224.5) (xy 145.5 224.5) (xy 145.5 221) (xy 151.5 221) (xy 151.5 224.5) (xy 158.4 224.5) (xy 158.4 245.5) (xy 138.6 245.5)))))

